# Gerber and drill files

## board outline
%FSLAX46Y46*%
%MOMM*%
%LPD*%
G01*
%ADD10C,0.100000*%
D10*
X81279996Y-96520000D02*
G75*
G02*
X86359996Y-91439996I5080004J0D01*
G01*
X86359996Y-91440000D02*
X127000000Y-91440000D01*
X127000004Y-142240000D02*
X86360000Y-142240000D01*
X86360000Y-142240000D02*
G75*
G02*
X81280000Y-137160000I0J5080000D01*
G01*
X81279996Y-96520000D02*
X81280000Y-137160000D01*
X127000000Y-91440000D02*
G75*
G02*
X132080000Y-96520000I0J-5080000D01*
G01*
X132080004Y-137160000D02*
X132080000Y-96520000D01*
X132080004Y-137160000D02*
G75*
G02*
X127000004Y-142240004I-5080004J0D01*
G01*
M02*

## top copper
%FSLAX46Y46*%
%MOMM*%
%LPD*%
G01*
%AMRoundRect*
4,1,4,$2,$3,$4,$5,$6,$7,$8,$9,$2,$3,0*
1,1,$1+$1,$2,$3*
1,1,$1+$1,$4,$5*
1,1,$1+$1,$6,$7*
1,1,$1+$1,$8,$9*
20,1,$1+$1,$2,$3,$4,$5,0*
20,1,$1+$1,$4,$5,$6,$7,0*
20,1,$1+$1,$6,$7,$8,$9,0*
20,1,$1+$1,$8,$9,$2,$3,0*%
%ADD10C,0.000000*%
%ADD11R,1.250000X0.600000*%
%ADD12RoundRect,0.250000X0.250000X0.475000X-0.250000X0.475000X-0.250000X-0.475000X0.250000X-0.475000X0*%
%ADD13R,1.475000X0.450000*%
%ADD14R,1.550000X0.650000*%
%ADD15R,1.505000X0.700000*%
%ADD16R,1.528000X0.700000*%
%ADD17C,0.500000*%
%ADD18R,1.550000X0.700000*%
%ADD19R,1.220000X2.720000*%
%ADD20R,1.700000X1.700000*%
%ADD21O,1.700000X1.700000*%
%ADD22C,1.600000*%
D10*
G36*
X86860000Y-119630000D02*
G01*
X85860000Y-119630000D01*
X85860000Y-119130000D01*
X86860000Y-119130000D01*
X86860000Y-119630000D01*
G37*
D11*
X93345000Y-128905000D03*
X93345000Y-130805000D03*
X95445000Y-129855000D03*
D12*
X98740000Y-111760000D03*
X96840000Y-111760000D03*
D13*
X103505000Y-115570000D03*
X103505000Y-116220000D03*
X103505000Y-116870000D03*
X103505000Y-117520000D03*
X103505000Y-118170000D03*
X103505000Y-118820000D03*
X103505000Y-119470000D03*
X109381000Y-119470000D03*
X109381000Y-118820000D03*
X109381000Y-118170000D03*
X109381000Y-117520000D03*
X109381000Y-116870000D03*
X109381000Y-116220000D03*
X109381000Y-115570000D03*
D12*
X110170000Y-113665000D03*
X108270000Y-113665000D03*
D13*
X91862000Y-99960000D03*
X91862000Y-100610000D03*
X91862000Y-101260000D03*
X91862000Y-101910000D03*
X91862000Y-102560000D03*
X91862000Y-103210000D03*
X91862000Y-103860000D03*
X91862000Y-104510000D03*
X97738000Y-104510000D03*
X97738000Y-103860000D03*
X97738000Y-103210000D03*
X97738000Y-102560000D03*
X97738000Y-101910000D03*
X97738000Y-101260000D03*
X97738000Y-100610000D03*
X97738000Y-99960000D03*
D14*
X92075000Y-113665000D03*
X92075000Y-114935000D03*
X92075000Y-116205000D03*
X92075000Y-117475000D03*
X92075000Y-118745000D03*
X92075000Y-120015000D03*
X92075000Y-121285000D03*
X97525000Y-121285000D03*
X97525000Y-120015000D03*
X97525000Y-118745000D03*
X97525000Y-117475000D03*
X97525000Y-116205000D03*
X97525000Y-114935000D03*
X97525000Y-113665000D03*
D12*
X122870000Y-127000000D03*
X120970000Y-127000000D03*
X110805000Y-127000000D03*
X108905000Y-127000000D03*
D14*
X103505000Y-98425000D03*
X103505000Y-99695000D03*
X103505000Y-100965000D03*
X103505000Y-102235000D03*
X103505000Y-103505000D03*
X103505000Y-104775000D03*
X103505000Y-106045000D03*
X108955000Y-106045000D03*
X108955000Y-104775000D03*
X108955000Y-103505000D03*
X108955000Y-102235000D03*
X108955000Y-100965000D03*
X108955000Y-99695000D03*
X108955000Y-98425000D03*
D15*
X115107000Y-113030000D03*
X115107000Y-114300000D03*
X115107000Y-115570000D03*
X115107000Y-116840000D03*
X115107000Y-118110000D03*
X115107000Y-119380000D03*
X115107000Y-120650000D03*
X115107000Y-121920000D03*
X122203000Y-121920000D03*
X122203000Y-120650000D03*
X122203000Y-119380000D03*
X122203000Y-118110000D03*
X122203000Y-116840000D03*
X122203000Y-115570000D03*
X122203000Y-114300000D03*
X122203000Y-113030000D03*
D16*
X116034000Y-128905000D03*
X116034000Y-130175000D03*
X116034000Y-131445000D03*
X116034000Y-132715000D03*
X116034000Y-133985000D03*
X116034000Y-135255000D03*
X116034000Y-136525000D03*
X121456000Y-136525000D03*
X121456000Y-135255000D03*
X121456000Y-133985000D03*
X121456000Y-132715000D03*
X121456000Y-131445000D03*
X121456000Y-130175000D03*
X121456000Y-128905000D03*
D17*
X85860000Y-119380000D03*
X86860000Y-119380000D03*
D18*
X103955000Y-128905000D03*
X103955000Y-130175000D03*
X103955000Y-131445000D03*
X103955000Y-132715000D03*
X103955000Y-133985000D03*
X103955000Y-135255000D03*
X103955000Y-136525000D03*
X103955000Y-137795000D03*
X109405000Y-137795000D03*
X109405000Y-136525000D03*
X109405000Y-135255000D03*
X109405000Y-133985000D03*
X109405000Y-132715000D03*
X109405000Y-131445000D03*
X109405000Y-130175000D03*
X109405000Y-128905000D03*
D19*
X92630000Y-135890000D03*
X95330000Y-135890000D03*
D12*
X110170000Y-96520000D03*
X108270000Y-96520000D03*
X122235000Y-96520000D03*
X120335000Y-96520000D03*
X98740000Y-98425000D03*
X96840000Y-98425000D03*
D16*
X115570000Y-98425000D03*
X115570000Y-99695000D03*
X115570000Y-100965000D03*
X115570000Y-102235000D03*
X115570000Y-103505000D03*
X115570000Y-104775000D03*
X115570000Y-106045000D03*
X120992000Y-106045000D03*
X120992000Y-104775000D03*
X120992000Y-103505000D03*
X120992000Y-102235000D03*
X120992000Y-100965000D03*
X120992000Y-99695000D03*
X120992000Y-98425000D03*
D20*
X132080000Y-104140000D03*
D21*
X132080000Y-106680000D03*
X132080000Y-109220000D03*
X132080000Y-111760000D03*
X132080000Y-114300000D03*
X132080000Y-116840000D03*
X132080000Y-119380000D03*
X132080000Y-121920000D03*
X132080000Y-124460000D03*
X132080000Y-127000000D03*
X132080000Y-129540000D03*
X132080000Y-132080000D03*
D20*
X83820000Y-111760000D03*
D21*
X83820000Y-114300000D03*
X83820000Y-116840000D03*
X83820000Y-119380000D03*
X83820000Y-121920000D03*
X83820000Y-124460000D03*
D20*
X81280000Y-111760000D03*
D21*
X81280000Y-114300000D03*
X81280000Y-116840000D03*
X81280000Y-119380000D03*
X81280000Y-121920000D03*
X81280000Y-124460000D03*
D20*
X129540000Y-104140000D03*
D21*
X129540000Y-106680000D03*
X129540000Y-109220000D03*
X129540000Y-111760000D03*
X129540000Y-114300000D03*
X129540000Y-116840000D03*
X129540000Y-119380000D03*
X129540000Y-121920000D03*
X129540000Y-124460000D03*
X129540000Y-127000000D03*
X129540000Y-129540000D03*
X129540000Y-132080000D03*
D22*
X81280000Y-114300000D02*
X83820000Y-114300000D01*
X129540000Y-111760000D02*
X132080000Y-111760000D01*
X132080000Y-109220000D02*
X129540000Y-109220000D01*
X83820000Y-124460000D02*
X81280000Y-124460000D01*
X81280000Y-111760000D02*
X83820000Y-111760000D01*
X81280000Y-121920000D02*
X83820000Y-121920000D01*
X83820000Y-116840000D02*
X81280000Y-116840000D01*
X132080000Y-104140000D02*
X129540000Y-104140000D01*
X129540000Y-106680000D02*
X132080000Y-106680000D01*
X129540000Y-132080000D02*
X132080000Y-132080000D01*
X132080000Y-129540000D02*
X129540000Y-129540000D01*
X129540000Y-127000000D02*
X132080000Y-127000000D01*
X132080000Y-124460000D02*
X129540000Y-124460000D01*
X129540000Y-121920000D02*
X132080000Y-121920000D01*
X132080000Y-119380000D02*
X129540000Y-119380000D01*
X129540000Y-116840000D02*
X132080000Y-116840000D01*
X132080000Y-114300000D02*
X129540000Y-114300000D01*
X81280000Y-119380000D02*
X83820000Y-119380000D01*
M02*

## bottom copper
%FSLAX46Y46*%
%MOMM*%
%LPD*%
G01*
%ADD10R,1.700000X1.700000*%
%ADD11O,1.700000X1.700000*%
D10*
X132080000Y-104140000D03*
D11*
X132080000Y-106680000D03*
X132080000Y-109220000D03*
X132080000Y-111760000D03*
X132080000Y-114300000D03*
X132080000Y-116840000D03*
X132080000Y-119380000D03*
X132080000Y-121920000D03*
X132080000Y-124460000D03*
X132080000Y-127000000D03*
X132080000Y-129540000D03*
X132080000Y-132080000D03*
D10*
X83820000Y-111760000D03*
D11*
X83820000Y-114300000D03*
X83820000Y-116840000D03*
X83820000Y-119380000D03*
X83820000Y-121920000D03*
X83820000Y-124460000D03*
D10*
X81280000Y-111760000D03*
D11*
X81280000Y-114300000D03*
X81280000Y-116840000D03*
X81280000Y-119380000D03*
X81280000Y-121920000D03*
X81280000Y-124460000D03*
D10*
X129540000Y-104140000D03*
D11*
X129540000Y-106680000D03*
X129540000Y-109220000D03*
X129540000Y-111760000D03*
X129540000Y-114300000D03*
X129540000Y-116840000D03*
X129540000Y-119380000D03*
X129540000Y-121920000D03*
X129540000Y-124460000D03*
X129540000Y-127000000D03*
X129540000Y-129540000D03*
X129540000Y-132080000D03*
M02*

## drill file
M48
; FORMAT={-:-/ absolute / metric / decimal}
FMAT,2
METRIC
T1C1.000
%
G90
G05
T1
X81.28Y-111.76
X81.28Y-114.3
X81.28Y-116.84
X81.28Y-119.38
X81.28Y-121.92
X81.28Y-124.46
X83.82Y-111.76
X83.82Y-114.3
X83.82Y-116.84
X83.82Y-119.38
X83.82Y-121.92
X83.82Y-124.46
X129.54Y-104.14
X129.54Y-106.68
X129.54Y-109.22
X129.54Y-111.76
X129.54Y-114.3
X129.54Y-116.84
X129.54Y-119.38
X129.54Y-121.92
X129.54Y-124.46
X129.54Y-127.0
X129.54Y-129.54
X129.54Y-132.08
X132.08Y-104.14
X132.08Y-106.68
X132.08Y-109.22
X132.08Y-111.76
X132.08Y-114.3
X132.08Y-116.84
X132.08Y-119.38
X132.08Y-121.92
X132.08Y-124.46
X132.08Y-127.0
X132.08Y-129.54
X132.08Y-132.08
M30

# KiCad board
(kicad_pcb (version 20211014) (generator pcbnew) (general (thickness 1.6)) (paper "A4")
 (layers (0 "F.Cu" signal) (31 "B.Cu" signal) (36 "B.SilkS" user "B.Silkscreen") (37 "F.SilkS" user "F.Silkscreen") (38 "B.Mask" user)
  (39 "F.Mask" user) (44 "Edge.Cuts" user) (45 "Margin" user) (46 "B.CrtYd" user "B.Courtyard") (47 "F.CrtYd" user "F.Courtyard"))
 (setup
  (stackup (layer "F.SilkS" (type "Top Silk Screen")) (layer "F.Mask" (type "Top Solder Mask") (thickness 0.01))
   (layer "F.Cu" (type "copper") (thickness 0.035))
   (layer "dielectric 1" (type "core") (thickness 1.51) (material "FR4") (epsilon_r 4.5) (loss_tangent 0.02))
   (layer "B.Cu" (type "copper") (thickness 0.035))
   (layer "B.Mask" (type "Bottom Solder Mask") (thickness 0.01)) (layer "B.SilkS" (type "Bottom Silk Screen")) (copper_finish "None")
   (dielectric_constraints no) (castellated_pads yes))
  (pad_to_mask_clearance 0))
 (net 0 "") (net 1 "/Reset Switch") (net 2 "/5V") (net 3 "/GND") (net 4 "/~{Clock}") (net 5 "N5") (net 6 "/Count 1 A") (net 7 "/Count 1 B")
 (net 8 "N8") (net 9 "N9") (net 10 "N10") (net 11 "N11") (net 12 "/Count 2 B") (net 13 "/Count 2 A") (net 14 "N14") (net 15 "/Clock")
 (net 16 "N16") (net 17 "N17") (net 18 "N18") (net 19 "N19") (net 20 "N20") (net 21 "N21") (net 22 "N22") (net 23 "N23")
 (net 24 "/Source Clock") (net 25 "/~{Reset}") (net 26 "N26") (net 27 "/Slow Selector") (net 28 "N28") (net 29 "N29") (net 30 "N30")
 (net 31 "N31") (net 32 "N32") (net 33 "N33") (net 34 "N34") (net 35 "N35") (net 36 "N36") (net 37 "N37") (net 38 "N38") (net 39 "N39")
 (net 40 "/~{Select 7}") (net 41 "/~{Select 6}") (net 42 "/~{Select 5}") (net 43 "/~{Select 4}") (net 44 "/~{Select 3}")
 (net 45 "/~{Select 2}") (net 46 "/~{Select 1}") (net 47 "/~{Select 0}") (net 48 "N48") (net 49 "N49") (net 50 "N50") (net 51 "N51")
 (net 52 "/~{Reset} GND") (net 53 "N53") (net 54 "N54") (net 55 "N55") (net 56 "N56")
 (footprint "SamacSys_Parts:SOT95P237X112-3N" (layer "F.Cu") (at 94.395 129.855)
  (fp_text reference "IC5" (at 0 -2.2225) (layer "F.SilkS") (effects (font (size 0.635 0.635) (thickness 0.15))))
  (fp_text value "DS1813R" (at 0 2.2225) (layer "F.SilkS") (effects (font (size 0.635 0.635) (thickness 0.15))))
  (pad "1" smd rect locked (at -1.05 -0.95 90) (size 0.6 1.25) (layers "F.Cu" "F.Paste" "F.Mask") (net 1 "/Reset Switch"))
  (pad "2" smd rect locked (at -1.05 0.95 90) (size 0.6 1.25) (layers "F.Cu" "F.Paste" "F.Mask") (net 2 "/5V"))
  (pad "3" smd rect locked (at 1.05 0 90) (size 0.6 1.25) (layers "F.Cu" "F.Paste" "F.Mask") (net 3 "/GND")))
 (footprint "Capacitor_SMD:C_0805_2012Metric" (layer "F.Cu") (at 97.79 111.76 180)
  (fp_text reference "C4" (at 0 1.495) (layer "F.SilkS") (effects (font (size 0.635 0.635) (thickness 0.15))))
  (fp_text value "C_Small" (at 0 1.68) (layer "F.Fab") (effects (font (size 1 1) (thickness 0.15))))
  (pad "1" smd roundrect (at -0.95 0 180) (size 1 1.45) (layers "F.Cu" "F.Paste" "F.Mask") (roundrect_rratio 0.25) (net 3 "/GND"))
  (pad "2" smd roundrect (at 0.95 0 180) (size 1 1.45) (layers "F.Cu" "F.Paste" "F.Mask") (roundrect_rratio 0.25) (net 2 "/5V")))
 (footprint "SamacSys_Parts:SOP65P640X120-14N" (layer "F.Cu") (at 106.443 117.52)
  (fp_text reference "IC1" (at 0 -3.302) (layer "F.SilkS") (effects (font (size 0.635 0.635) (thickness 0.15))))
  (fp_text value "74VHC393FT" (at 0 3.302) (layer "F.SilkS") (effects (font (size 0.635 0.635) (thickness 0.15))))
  (pad "1" smd rect (at -2.938 -1.95 90) (size 0.45 1.475) (layers "F.Cu" "F.Paste" "F.Mask") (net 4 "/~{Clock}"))
  (pad "2" smd rect (at -2.938 -1.3 90) (size 0.45 1.475) (layers "F.Cu" "F.Paste" "F.Mask") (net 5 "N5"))
  (pad "3" smd rect (at -2.938 -0.65 90) (size 0.45 1.475) (layers "F.Cu" "F.Paste" "F.Mask") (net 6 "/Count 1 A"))
  (pad "4" smd rect (at -2.938 0 90) (size 0.45 1.475) (layers "F.Cu" "F.Paste" "F.Mask") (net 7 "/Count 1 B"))
  (pad "5" smd rect (at -2.938 0.65 90) (size 0.45 1.475) (layers "F.Cu" "F.Paste" "F.Mask") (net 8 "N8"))
  (pad "6" smd rect (at -2.938 1.3 90) (size 0.45 1.475) (layers "F.Cu" "F.Paste" "F.Mask") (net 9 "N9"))
  (pad "7" smd rect (at -2.938 1.95 90) (size 0.45 1.475) (layers "F.Cu" "F.Paste" "F.Mask") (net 3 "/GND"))
  (pad "8" smd rect (at 2.938 1.95 90) (size 0.45 1.475) (layers "F.Cu" "F.Paste" "F.Mask") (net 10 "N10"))
  (pad "9" smd rect (at 2.938 1.3 90) (size 0.45 1.475) (layers "F.Cu" "F.Paste" "F.Mask") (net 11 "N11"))
  (pad "10" smd rect (at 2.938 0.65 90) (size 0.45 1.475) (layers "F.Cu" "F.Paste" "F.Mask") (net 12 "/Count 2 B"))
  (pad "11" smd rect (at 2.938 0 90) (size 0.45 1.475) (layers "F.Cu" "F.Paste" "F.Mask") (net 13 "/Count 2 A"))
  (pad "12" smd rect (at 2.938 -0.65 90) (size 0.45 1.475) (layers "F.Cu" "F.Paste" "F.Mask") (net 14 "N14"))
  (pad "13" smd rect (at 2.938 -1.3 90) (size 0.45 1.475) (layers "F.Cu" "F.Paste" "F.Mask") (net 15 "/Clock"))
  (pad "14" smd rect (at 2.938 -1.95 90) (size 0.45 1.475) (layers "F.Cu" "F.Paste" "F.Mask") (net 2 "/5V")))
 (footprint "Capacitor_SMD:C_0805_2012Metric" (layer "F.Cu") (at 109.22 113.665 180)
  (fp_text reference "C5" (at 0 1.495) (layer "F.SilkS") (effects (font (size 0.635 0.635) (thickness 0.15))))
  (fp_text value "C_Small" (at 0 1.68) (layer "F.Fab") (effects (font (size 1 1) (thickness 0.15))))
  (pad "1" smd roundrect (at -0.95 0 180) (size 1 1.45) (layers "F.Cu" "F.Paste" "F.Mask") (roundrect_rratio 0.25) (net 3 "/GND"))
  (pad "2" smd roundrect (at 0.95 0 180) (size 1 1.45) (layers "F.Cu" "F.Paste" "F.Mask") (roundrect_rratio 0.25) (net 2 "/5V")))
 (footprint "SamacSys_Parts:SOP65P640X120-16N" (layer "F.Cu") (at 94.8 102.235)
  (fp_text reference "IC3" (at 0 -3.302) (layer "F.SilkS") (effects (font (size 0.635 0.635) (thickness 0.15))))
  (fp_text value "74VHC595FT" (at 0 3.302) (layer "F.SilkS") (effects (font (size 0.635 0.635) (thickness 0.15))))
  (pad "1" smd rect (at -2.938 -2.275 90) (size 0.45 1.475) (layers "F.Cu" "F.Paste" "F.Mask") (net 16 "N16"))
  (pad "2" smd rect (at -2.938 -1.625 90) (size 0.45 1.475) (layers "F.Cu" "F.Paste" "F.Mask") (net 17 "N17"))
  (pad "3" smd rect (at -2.938 -0.975 90) (size 0.45 1.475) (layers "F.Cu" "F.Paste" "F.Mask") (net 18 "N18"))
  (pad "4" smd rect (at -2.938 -0.325 90) (size 0.45 1.475) (layers "F.Cu" "F.Paste" "F.Mask") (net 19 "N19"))
  (pad "5" smd rect (at -2.938 0.325 90) (size 0.45 1.475) (layers "F.Cu" "F.Paste" "F.Mask") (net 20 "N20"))
  (pad "6" smd rect (at -2.938 0.975 90) (size 0.45 1.475) (layers "F.Cu" "F.Paste" "F.Mask") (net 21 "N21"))
  (pad "7" smd rect (at -2.938 1.625 90) (size 0.45 1.475) (layers "F.Cu" "F.Paste" "F.Mask") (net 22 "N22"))
  (pad "8" smd rect (at -2.938 2.275 90) (size 0.45 1.475) (layers "F.Cu" "F.Paste" "F.Mask") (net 3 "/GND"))
  (pad "9" smd rect (at 2.938 2.275 90) (size 0.45 1.475) (layers "F.Cu" "F.Paste" "F.Mask") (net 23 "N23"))
  (pad "10" smd rect (at 2.938 1.625 90) (size 0.45 1.475) (layers "F.Cu" "F.Paste" "F.Mask") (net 1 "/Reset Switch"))
  (pad "11" smd rect (at 2.938 0.975 90) (size 0.45 1.475) (layers "F.Cu" "F.Paste" "F.Mask") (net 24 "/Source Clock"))
  (pad "12" smd rect (at 2.938 0.325 90) (size 0.45 1.475) (layers "F.Cu" "F.Paste" "F.Mask") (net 24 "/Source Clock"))
  (pad "13" smd rect (at 2.938 -0.325 90) (size 0.45 1.475) (layers "F.Cu" "F.Paste" "F.Mask") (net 3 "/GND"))
  (pad "14" smd rect (at 2.938 -0.975 90) (size 0.45 1.475) (layers "F.Cu" "F.Paste" "F.Mask") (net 1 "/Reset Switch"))
  (pad "15" smd rect (at 2.938 -1.625 90) (size 0.45 1.475) (layers "F.Cu" "F.Paste" "F.Mask") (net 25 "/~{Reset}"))
  (pad "16" smd rect (at 2.938 -2.275 90) (size 0.45 1.475) (layers "F.Cu" "F.Paste" "F.Mask") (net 2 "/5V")))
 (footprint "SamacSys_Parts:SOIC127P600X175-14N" (layer "F.Cu") (at 94.8 117.475)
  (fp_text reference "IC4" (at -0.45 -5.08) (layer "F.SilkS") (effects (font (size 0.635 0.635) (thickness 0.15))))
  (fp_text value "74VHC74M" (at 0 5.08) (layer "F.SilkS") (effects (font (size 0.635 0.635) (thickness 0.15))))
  (pad "1" smd rect locked (at -2.725 -3.81 90) (size 0.65 1.55) (layers "F.Cu" "F.Paste" "F.Mask") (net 19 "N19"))
  (pad "2" smd rect locked (at -2.725 -2.54 90) (size 0.65 1.55) (layers "F.Cu" "F.Paste" "F.Mask") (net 4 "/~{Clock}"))
  (pad "3" smd rect locked (at -2.725 -1.27 90) (size 0.65 1.55) (layers "F.Cu" "F.Paste" "F.Mask") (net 24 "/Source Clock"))
  (pad "4" smd rect locked (at -2.725 0 90) (size 0.65 1.55) (layers "F.Cu" "F.Paste" "F.Mask") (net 2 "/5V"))
  (pad "5" smd rect locked (at -2.725 1.27 90) (size 0.65 1.55) (layers "F.Cu" "F.Paste" "F.Mask") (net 15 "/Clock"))
  (pad "6" smd rect locked (at -2.725 2.54 90) (size 0.65 1.55) (layers "F.Cu" "F.Paste" "F.Mask") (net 4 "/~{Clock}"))
  (pad "7" smd rect locked (at -2.725 3.81 90) (size 0.65 1.55) (layers "F.Cu" "F.Paste" "F.Mask") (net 3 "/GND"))
  (pad "8" smd rect locked (at 2.725 3.81 90) (size 0.65 1.55) (layers "F.Cu" "F.Paste" "F.Mask") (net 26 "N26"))
  (pad "9" smd rect locked (at 2.725 2.54 90) (size 0.65 1.55) (layers "F.Cu" "F.Paste" "F.Mask") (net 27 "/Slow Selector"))
  (pad "10" smd rect locked (at 2.725 1.27 90) (size 0.65 1.55) (layers "F.Cu" "F.Paste" "F.Mask") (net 2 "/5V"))
  (pad "11" smd rect locked (at 2.725 0 90) (size 0.65 1.55) (layers "F.Cu" "F.Paste" "F.Mask") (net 9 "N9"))
  (pad "12" smd rect locked (at 2.725 -1.27 90) (size 0.65 1.55) (layers "F.Cu" "F.Paste" "F.Mask") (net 26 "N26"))
  (pad "13" smd rect locked (at 2.725 -2.54 90) (size 0.65 1.55) (layers "F.Cu" "F.Paste" "F.Mask") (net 19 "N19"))
  (pad "14" smd rect locked (at 2.725 -3.81 90) (size 0.65 1.55) (layers "F.Cu" "F.Paste" "F.Mask") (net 2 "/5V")))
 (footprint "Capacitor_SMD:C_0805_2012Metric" (layer "F.Cu") (at 121.92 127 180)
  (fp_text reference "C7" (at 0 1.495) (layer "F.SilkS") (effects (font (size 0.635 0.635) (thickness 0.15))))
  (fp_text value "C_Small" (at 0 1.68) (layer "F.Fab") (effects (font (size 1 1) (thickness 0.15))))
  (pad "1" smd roundrect (at -0.95 0 180) (size 1 1.45) (layers "F.Cu" "F.Paste" "F.Mask") (roundrect_rratio 0.25) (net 3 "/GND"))
  (pad "2" smd roundrect (at 0.95 0 180) (size 1 1.45) (layers "F.Cu" "F.Paste" "F.Mask") (roundrect_rratio 0.25) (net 2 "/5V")))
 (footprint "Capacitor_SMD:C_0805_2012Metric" (layer "F.Cu") (at 109.855 127 180)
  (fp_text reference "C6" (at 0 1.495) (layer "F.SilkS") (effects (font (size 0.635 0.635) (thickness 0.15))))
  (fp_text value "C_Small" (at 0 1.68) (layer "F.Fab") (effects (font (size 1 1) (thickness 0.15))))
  (pad "1" smd roundrect (at -0.95 0 180) (size 1 1.45) (layers "F.Cu" "F.Paste" "F.Mask") (roundrect_rratio 0.25) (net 3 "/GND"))
  (pad "2" smd roundrect (at 0.95 0 180) (size 1 1.45) (layers "F.Cu" "F.Paste" "F.Mask") (roundrect_rratio 0.25) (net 2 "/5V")))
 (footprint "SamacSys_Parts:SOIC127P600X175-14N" (layer "F.Cu") (at 106.23 102.235)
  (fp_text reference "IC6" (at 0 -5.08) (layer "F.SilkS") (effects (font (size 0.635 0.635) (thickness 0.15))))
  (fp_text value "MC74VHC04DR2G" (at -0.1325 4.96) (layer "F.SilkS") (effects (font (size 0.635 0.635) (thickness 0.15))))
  (pad "1" smd rect locked (at -2.725 -3.81 90) (size 0.65 1.55) (layers "F.Cu" "F.Paste" "F.Mask") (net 21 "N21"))
  (pad "2" smd rect locked (at -2.725 -2.54 90) (size 0.65 1.55) (layers "F.Cu" "F.Paste" "F.Mask") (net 5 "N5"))
  (pad "3" smd rect locked (at -2.725 -1.27 90) (size 0.65 1.55) (layers "F.Cu" "F.Paste" "F.Mask") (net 22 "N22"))
  (pad "4" smd rect locked (at -2.725 0 90) (size 0.65 1.55) (layers "F.Cu" "F.Paste" "F.Mask") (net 14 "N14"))
  (pad "5" smd rect locked (at -2.725 1.27 90) (size 0.65 1.55) (layers "F.Cu" "F.Paste" "F.Mask") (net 3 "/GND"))
  (pad "6" smd rect locked (at -2.725 2.54 90) (size 0.65 1.55) (layers "F.Cu" "F.Paste" "F.Mask") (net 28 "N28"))
  (pad "7" smd rect locked (at -2.725 3.81 90) (size 0.65 1.55) (layers "F.Cu" "F.Paste" "F.Mask") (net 3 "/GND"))
  (pad "8" smd rect locked (at 2.725 3.81 90) (size 0.65 1.55) (layers "F.Cu" "F.Paste" "F.Mask") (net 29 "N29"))
  (pad "9" smd rect locked (at 2.725 2.54 90) (size 0.65 1.55) (layers "F.Cu" "F.Paste" "F.Mask") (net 3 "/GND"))
  (pad "10" smd rect locked (at 2.725 1.27 90) (size 0.65 1.55) (layers "F.Cu" "F.Paste" "F.Mask") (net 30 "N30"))
  (pad "11" smd rect locked (at 2.725 0 90) (size 0.65 1.55) (layers "F.Cu" "F.Paste" "F.Mask") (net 3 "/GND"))
  (pad "12" smd rect locked (at 2.725 -1.27 90) (size 0.65 1.55) (layers "F.Cu" "F.Paste" "F.Mask") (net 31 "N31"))
  (pad "13" smd rect locked (at 2.725 -2.54 90) (size 0.65 1.55) (layers "F.Cu" "F.Paste" "F.Mask") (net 3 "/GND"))
  (pad "14" smd rect locked (at 2.725 -3.81 90) (size 0.65 1.55) (layers "F.Cu" "F.Paste" "F.Mask") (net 2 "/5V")))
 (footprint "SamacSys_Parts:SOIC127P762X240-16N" (layer "F.Cu") (at 118.655 117.475)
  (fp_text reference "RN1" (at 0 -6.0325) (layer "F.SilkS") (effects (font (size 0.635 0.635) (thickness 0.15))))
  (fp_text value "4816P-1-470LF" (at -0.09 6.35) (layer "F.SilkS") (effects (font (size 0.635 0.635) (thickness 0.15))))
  (pad "1" smd rect (at -3.548 -4.445 90) (size 0.7 1.505) (layers "F.Cu" "F.Paste" "F.Mask") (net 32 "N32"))
  (pad "2" smd rect (at -3.548 -3.175 90) (size 0.7 1.505) (layers "F.Cu" "F.Paste" "F.Mask") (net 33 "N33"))
  (pad "3" smd rect (at -3.548 -1.905 90) (size 0.7 1.505) (layers "F.Cu" "F.Paste" "F.Mask") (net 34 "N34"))
  (pad "4" smd rect (at -3.548 -0.635 90) (size 0.7 1.505) (layers "F.Cu" "F.Paste" "F.Mask") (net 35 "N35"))
  (pad "5" smd rect (at -3.548 0.635 90) (size 0.7 1.505) (layers "F.Cu" "F.Paste" "F.Mask") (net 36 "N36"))
  (pad "6" smd rect (at -3.548 1.905 90) (size 0.7 1.505) (layers "F.Cu" "F.Paste" "F.Mask") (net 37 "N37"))
  (pad "7" smd rect (at -3.548 3.175 90) (size 0.7 1.505) (layers "F.Cu" "F.Paste" "F.Mask") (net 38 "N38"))
  (pad "8" smd rect (at -3.548 4.445 90) (size 0.7 1.505) (layers "F.Cu" "F.Paste" "F.Mask") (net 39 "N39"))
  (pad "9" smd rect (at 3.548 4.445 90) (size 0.7 1.505) (layers "F.Cu" "F.Paste" "F.Mask") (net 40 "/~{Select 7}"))
  (pad "10" smd rect (at 3.548 3.175 90) (size 0.7 1.505) (layers "F.Cu" "F.Paste" "F.Mask") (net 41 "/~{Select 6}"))
  (pad "11" smd rect (at 3.548 1.905 90) (size 0.7 1.505) (layers "F.Cu" "F.Paste" "F.Mask") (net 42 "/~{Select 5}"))
  (pad "12" smd rect (at 3.548 0.635 90) (size 0.7 1.505) (layers "F.Cu" "F.Paste" "F.Mask") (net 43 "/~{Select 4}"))
  (pad "13" smd rect (at 3.548 -0.635 90) (size 0.7 1.505) (layers "F.Cu" "F.Paste" "F.Mask") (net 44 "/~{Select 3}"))
  (pad "14" smd rect (at 3.548 -1.905 90) (size 0.7 1.505) (layers "F.Cu" "F.Paste" "F.Mask") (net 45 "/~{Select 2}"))
  (pad "15" smd rect (at 3.548 -3.175 90) (size 0.7 1.505) (layers "F.Cu" "F.Paste" "F.Mask") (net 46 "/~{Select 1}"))
  (pad "16" smd rect (at 3.548 -4.445 90) (size 0.7 1.505) (layers "F.Cu" "F.Paste" "F.Mask") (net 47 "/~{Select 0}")))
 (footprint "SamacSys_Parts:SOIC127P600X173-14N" (layer "F.Cu") (at 118.745 132.715)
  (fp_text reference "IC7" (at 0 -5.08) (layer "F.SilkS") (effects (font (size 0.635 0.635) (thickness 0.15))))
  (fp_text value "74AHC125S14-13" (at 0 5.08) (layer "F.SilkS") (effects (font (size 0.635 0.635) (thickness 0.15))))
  (pad "1" smd rect (at -2.711 -3.81 90) (size 0.7 1.528) (layers "F.Cu" "F.Paste" "F.Mask") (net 3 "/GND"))
  (pad "2" smd rect (at -2.711 -2.54 90) (size 0.7 1.528) (layers "F.Cu" "F.Paste" "F.Mask") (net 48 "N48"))
  (pad "3" smd rect (at -2.711 -1.27 90) (size 0.7 1.528) (layers "F.Cu" "F.Paste" "F.Mask") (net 33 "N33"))
  (pad "4" smd rect (at -2.711 0 90) (size 0.7 1.528) (layers "F.Cu" "F.Paste" "F.Mask") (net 3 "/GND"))
  (pad "5" smd rect (at -2.711 1.27 90) (size 0.7 1.528) (layers "F.Cu" "F.Paste" "F.Mask") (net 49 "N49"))
  (pad "6" smd rect (at -2.711 2.54 90) (size 0.7 1.528) (layers "F.Cu" "F.Paste" "F.Mask") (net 35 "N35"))
  (pad "7" smd rect (at -2.711 3.81 90) (size 0.7 1.528) (layers "F.Cu" "F.Paste" "F.Mask") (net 3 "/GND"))
  (pad "8" smd rect (at 2.711 3.81 90) (size 0.7 1.528) (layers "F.Cu" "F.Paste" "F.Mask") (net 37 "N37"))
  (pad "9" smd rect (at 2.711 2.54 90) (size 0.7 1.528) (layers "F.Cu" "F.Paste" "F.Mask") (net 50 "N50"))
  (pad "10" smd rect (at 2.711 1.27 90) (size 0.7 1.528) (layers "F.Cu" "F.Paste" "F.Mask") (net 3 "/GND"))
  (pad "11" smd rect (at 2.711 0 90) (size 0.7 1.528) (layers "F.Cu" "F.Paste" "F.Mask") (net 39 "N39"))
  (pad "12" smd rect (at 2.711 -1.27 90) (size 0.7 1.528) (layers "F.Cu" "F.Paste" "F.Mask") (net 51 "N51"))
  (pad "13" smd rect (at 2.711 -2.54 90) (size 0.7 1.528) (layers "F.Cu" "F.Paste" "F.Mask") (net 3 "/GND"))
  (pad "14" smd rect (at 2.711 -3.81 90) (size 0.7 1.528) (layers "F.Cu" "F.Paste" "F.Mask") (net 2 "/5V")))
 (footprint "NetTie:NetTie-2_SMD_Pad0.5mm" (layer "F.Cu") (at 86.36 119.38)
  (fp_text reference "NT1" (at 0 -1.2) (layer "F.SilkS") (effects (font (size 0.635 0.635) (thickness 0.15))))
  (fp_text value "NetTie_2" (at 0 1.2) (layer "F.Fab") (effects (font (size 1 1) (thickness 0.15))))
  (fp_poly (pts (xy -0.5 -0.25) (xy 0.5 -0.25) (xy 0.5 0.25) (xy -0.5 0.25)) (layer "F.Cu") (width 0) (fill solid))
  (pad "1" smd circle (at -0.5 0) (size 0.5 0.5) (layers "F.Cu") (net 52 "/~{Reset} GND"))
  (pad "2" smd circle (at 0.5 0) (size 0.5 0.5) (layers "F.Cu") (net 3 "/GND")))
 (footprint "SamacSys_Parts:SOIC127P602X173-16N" (layer "F.Cu") (at 106.68 133.35)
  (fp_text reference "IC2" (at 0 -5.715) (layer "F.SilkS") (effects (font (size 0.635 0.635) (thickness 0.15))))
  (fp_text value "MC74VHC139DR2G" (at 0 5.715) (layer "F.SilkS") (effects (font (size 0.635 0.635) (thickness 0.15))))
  (pad "1" smd rect (at -2.725 -4.445 90) (size 0.7 1.55) (layers "F.Cu" "F.Paste" "F.Mask") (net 3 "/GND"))
  (pad "2" smd rect (at -2.725 -3.175 90) (size 0.7 1.55) (layers "F.Cu" "F.Paste" "F.Mask") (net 6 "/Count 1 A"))
  (pad "3" smd rect (at -2.725 -1.905 90) (size 0.7 1.55) (layers "F.Cu" "F.Paste" "F.Mask") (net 7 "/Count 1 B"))
  (pad "4" smd rect (at -2.725 -0.635 90) (size 0.7 1.55) (layers "F.Cu" "F.Paste" "F.Mask") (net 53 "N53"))
  (pad "5" smd rect (at -2.725 0.635 90) (size 0.7 1.55) (layers "F.Cu" "F.Paste" "F.Mask") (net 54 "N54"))
  (pad "6" smd rect (at -2.725 1.905 90) (size 0.7 1.55) (layers "F.Cu" "F.Paste" "F.Mask") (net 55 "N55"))
  (pad "7" smd rect (at -2.725 3.175 90) (size 0.7 1.55) (layers "F.Cu" "F.Paste" "F.Mask") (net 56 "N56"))
  (pad "8" smd rect (at -2.725 4.445 90) (size 0.7 1.55) (layers "F.Cu" "F.Paste" "F.Mask") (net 3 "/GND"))
  (pad "9" smd rect (at 2.725 4.445 90) (size 0.7 1.55) (layers "F.Cu" "F.Paste" "F.Mask") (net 51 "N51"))
  (pad "10" smd rect (at 2.725 3.175 90) (size 0.7 1.55) (layers "F.Cu" "F.Paste" "F.Mask") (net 50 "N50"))
  (pad "11" smd rect (at 2.725 1.905 90) (size 0.7 1.55) (layers "F.Cu" "F.Paste" "F.Mask") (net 49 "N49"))
  (pad "12" smd rect (at 2.725 0.635 90) (size 0.7 1.55) (layers "F.Cu" "F.Paste" "F.Mask") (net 48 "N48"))
  (pad "13" smd rect (at 2.725 -0.635 90) (size 0.7 1.55) (layers "F.Cu" "F.Paste" "F.Mask") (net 12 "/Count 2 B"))
  (pad "14" smd rect (at 2.725 -1.905 90) (size 0.7 1.55) (layers "F.Cu" "F.Paste" "F.Mask") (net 13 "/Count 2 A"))
  (pad "15" smd rect (at 2.725 -3.175 90) (size 0.7 1.55) (layers "F.Cu" "F.Paste" "F.Mask") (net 3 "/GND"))
  (pad "16" smd rect (at 2.725 -4.445 90) (size 0.7 1.55) (layers "F.Cu" "F.Paste" "F.Mask") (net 2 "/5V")))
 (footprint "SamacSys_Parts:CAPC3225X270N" (layer "F.Cu") (at 93.98 135.89)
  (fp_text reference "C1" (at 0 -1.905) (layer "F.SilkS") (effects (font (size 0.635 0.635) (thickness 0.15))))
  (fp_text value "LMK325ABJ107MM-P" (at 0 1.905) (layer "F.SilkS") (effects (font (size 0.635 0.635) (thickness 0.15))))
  (pad "1" smd rect locked (at -1.35 0) (size 1.22 2.72) (layers "F.Cu" "F.Paste" "F.Mask") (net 2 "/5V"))
  (pad "2" smd rect locked (at 1.35 0) (size 1.22 2.72) (layers "F.Cu" "F.Paste" "F.Mask") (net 3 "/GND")))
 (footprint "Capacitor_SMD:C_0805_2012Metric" (layer "F.Cu") (at 109.22 96.52 180)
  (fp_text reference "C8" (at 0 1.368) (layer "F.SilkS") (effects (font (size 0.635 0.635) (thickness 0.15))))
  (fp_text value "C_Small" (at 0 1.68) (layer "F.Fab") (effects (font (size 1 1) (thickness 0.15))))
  (pad "1" smd roundrect (at -0.95 0 180) (size 1 1.45) (layers "F.Cu" "F.Paste" "F.Mask") (roundrect_rratio 0.25) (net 3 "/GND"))
  (pad "2" smd roundrect (at 0.95 0 180) (size 1 1.45) (layers "F.Cu" "F.Paste" "F.Mask") (roundrect_rratio 0.25) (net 2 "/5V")))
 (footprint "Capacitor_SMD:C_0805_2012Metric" (layer "F.Cu") (at 121.285 96.52 180)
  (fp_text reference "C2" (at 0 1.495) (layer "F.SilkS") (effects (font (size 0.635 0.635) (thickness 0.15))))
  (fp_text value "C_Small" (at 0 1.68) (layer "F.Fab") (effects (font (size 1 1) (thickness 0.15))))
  (pad "1" smd roundrect (at -0.95 0 180) (size 1 1.45) (layers "F.Cu" "F.Paste" "F.Mask") (roundrect_rratio 0.25) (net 3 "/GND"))
  (pad "2" smd roundrect (at 0.95 0 180) (size 1 1.45) (layers "F.Cu" "F.Paste" "F.Mask") (roundrect_rratio 0.25) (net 2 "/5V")))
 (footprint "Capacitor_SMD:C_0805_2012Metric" (layer "F.Cu") (at 97.79 98.425 180)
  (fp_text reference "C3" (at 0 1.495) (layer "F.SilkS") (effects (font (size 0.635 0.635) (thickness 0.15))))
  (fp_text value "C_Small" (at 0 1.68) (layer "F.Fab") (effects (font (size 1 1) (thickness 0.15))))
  (pad "1" smd roundrect (at -0.95 0 180) (size 1 1.45) (layers "F.Cu" "F.Paste" "F.Mask") (roundrect_rratio 0.25) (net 3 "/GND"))
  (pad "2" smd roundrect (at 0.95 0 180) (size 1 1.45) (layers "F.Cu" "F.Paste" "F.Mask") (roundrect_rratio 0.25) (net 2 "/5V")))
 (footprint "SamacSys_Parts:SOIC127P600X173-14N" (layer "F.Cu") (at 118.281 102.235)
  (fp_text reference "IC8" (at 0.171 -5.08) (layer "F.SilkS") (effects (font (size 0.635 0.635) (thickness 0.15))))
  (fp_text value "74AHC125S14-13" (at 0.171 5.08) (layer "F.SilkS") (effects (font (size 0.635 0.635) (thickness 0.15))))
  (pad "1" smd rect (at -2.711 -3.81 90) (size 0.7 1.528) (layers "F.Cu" "F.Paste" "F.Mask") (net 3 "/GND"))
  (pad "2" smd rect (at -2.711 -2.54 90) (size 0.7 1.528) (layers "F.Cu" "F.Paste" "F.Mask") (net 53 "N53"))
  (pad "3" smd rect (at -2.711 -1.27 90) (size 0.7 1.528) (layers "F.Cu" "F.Paste" "F.Mask") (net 32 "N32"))
  (pad "4" smd rect (at -2.711 0 90) (size 0.7 1.528) (layers "F.Cu" "F.Paste" "F.Mask") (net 3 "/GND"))
  (pad "5" smd rect (at -2.711 1.27 90) (size 0.7 1.528) (layers "F.Cu" "F.Paste" "F.Mask") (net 54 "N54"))
  (pad "6" smd rect (at -2.711 2.54 90) (size 0.7 1.528) (layers "F.Cu" "F.Paste" "F.Mask") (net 34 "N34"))
  (pad "7" smd rect (at -2.711 3.81 90) (size 0.7 1.528) (layers "F.Cu" "F.Paste" "F.Mask") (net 3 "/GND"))
  (pad "8" smd rect (at 2.711 3.81 90) (size 0.7 1.528) (layers "F.Cu" "F.Paste" "F.Mask") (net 36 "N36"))
  (pad "9" smd rect (at 2.711 2.54 90) (size 0.7 1.528) (layers "F.Cu" "F.Paste" "F.Mask") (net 55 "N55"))
  (pad "10" smd rect (at 2.711 1.27 90) (size 0.7 1.528) (layers "F.Cu" "F.Paste" "F.Mask") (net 3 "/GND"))
  (pad "11" smd rect (at 2.711 0 90) (size 0.7 1.528) (layers "F.Cu" "F.Paste" "F.Mask") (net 38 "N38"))
  (pad "12" smd rect (at 2.711 -1.27 90) (size 0.7 1.528) (layers "F.Cu" "F.Paste" "F.Mask") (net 56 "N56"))
  (pad "13" smd rect (at 2.711 -2.54 90) (size 0.7 1.528) (layers "F.Cu" "F.Paste" "F.Mask") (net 3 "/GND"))
  (pad "14" smd rect (at 2.711 -3.81 90) (size 0.7 1.528) (layers "F.Cu" "F.Paste" "F.Mask") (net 2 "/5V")))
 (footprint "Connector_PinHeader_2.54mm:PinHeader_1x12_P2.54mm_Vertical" (layer "B.Cu") (at 132.08 104.14 180)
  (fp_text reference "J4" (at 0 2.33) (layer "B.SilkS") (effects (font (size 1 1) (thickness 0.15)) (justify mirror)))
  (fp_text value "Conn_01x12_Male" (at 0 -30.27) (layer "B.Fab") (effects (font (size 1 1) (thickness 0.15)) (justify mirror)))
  (pad "1" thru_hole rect (at 0 0 180) (size 1.7 1.7) (drill 1) (layers *.Cu *.Mask) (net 25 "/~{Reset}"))
  (pad "2" thru_hole oval (at 0 -2.54 180) (size 1.7 1.7) (drill 1) (layers *.Cu *.Mask) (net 27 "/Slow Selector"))
  (pad "3" thru_hole oval (at 0 -5.08 180) (size 1.7 1.7) (drill 1) (layers *.Cu *.Mask) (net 15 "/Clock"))
  (pad "4" thru_hole oval (at 0 -7.62 180) (size 1.7 1.7) (drill 1) (layers *.Cu *.Mask) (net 4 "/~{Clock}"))
  (pad "5" thru_hole oval (at 0 -10.16 180) (size 1.7 1.7) (drill 1) (layers *.Cu *.Mask) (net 47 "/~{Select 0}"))
  (pad "6" thru_hole oval (at 0 -12.7 180) (size 1.7 1.7) (drill 1) (layers *.Cu *.Mask) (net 46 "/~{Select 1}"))
  (pad "7" thru_hole oval (at 0 -15.24 180) (size 1.7 1.7) (drill 1) (layers *.Cu *.Mask) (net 45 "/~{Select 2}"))
  (pad "8" thru_hole oval (at 0 -17.78 180) (size 1.7 1.7) (drill 1) (layers *.Cu *.Mask) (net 44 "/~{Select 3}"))
  (pad "9" thru_hole oval (at 0 -20.32 180) (size 1.7 1.7) (drill 1) (layers *.Cu *.Mask) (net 43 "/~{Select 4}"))
  (pad "10" thru_hole oval (at 0 -22.86 180) (size 1.7 1.7) (drill 1) (layers *.Cu *.Mask) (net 42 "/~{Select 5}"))
  (pad "11" thru_hole oval (at 0 -25.4 180) (size 1.7 1.7) (drill 1) (layers *.Cu *.Mask) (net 41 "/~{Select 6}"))
  (pad "12" thru_hole oval (at 0 -27.94 180) (size 1.7 1.7) (drill 1) (layers *.Cu *.Mask) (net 40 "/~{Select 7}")))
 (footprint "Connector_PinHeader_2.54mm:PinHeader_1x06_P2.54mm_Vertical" (layer "B.Cu") (at 83.82 111.76 180)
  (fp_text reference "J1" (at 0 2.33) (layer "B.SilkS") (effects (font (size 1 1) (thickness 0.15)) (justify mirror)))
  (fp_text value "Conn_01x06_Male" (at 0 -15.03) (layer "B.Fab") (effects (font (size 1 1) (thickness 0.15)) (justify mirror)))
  (pad "1" thru_hole rect (at 0 0 180) (size 1.7 1.7) (drill 1) (layers *.Cu *.Mask) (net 3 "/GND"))
  (pad "2" thru_hole oval (at 0 -2.54 180) (size 1.7 1.7) (drill 1) (layers *.Cu *.Mask) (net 2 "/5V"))
  (pad "3" thru_hole oval (at 0 -5.08 180) (size 1.7 1.7) (drill 1) (layers *.Cu *.Mask) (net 24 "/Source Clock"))
  (pad "4" thru_hole oval (at 0 -7.62 180) (size 1.7 1.7) (drill 1) (layers *.Cu *.Mask) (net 52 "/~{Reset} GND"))
  (pad "5" thru_hole oval (at 0 -10.16 180) (size 1.7 1.7) (drill 1) (layers *.Cu *.Mask) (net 1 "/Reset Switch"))
  (pad "6" thru_hole oval (at 0 -12.7 180) (size 1.7 1.7) (drill 1) (layers *.Cu *.Mask) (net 3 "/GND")))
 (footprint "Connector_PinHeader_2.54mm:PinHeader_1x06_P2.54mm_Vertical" (layer "B.Cu") (at 81.28 111.76 180)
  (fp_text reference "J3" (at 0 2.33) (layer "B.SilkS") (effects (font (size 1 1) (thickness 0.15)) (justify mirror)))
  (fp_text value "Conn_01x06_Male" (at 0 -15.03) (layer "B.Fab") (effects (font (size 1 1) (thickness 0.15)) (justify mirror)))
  (pad "1" thru_hole rect (at 0 0 180) (size 1.7 1.7) (drill 1) (layers *.Cu *.Mask) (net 3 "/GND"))
  (pad "2" thru_hole oval (at 0 -2.54 180) (size 1.7 1.7) (drill 1) (layers *.Cu *.Mask) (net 2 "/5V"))
  (pad "3" thru_hole oval (at 0 -5.08 180) (size 1.7 1.7) (drill 1) (layers *.Cu *.Mask) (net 24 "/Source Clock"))
  (pad "4" thru_hole oval (at 0 -7.62 180) (size 1.7 1.7) (drill 1) (layers *.Cu *.Mask) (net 52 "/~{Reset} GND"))
  (pad "5" thru_hole oval (at 0 -10.16 180) (size 1.7 1.7) (drill 1) (layers *.Cu *.Mask) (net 1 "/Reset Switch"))
  (pad "6" thru_hole oval (at 0 -12.7 180) (size 1.7 1.7) (drill 1) (layers *.Cu *.Mask) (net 3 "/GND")))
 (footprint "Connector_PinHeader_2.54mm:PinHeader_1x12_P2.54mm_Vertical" (layer "B.Cu") (at 129.54 104.14 180)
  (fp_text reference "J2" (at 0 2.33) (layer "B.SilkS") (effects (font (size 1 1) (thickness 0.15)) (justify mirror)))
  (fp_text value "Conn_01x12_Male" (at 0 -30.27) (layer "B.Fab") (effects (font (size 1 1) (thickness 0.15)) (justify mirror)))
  (pad "1" thru_hole rect (at 0 0 180) (size 1.7 1.7) (drill 1) (layers *.Cu *.Mask) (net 25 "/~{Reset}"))
  (pad "2" thru_hole oval (at 0 -2.54 180) (size 1.7 1.7) (drill 1) (layers *.Cu *.Mask) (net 27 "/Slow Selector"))
  (pad "3" thru_hole oval (at 0 -5.08 180) (size 1.7 1.7) (drill 1) (layers *.Cu *.Mask) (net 15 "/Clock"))
  (pad "4" thru_hole oval (at 0 -7.62 180) (size 1.7 1.7) (drill 1) (layers *.Cu *.Mask) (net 4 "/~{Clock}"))
  (pad "5" thru_hole oval (at 0 -10.16 180) (size 1.7 1.7) (drill 1) (layers *.Cu *.Mask) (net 47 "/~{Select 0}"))
  (pad "6" thru_hole oval (at 0 -12.7 180) (size 1.7 1.7) (drill 1) (layers *.Cu *.Mask) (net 46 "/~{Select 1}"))
  (pad "7" thru_hole oval (at 0 -15.24 180) (size 1.7 1.7) (drill 1) (layers *.Cu *.Mask) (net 45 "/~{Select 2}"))
  (pad "8" thru_hole oval (at 0 -17.78 180) (size 1.7 1.7) (drill 1) (layers *.Cu *.Mask) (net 44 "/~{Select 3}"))
  (pad "9" thru_hole oval (at 0 -20.32 180) (size 1.7 1.7) (drill 1) (layers *.Cu *.Mask) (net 43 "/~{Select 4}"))
  (pad "10" thru_hole oval (at 0 -22.86 180) (size 1.7 1.7) (drill 1) (layers *.Cu *.Mask) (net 42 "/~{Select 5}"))
  (pad "11" thru_hole oval (at 0 -25.4 180) (size 1.7 1.7) (drill 1) (layers *.Cu *.Mask) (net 41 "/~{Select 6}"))
  (pad "12" thru_hole oval (at 0 -27.94 180) (size 1.7 1.7) (drill 1) (layers *.Cu *.Mask) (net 40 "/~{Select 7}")))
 (gr_arc (start 81.279996 96.52) (mid 82.767894 92.927898) (end 86.359996 91.44) (layer "Edge.Cuts") (width 0.1))
 (gr_line (start 86.359996 91.44) (end 127 91.44) (layer "Edge.Cuts") (width 0.1))
 (gr_line (start 127.000004 142.24) (end 86.36 142.24) (layer "Edge.Cuts") (width 0.1))
 (gr_arc (start 86.36 142.24) (mid 82.767898 140.752102) (end 81.28 137.16) (layer "Edge.Cuts") (width 0.1))
 (gr_line (start 81.279996 96.52) (end 81.28 137.16) (layer "Edge.Cuts") (width 0.1))
 (gr_arc (start 127 91.44) (mid 130.592102 92.927898) (end 132.08 96.52) (layer "Edge.Cuts") (width 0.1))
 (gr_line (start 132.080004 137.16) (end 132.08 96.52) (layer "Edge.Cuts") (width 0.1))
 (gr_arc (start 132.080004 137.16) (mid 130.592106 140.752102) (end 127.000004 142.24) (layer "Edge.Cuts") (width 0.1))
 (segment (start 81.28 114.3) (end 83.82 114.3) (width 1.6) (layer "F.Cu") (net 2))
 (segment (start 129.54 111.76) (end 132.08 111.76) (width 1.6) (layer "F.Cu") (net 4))
 (segment (start 132.08 109.22) (end 129.54 109.22) (width 1.6) (layer "F.Cu") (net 15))
 (segment (start 83.82 124.46) (end 81.28 124.46) (width 1.6) (layer "F.Cu") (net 3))
 (segment (start 81.28 111.76) (end 83.82 111.76) (width 1.6) (layer "F.Cu") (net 3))
 (segment (start 81.28 121.92) (end 83.82 121.92) (width 1.6) (layer "F.Cu") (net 1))
 (segment (start 83.82 116.84) (end 81.28 116.84) (width 1.6) (layer "F.Cu") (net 24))
 (segment (start 132.08 104.14) (end 129.54 104.14) (width 1.6) (layer "F.Cu") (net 25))
 (segment (start 129.54 106.68) (end 132.08 106.68) (width 1.6) (layer "F.Cu") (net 27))
 (segment (start 129.54 132.08) (end 132.08 132.08) (width 1.6) (layer "F.Cu") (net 40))
 (segment (start 132.08 129.54) (end 129.54 129.54) (width 1.6) (layer "F.Cu") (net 41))
 (segment (start 129.54 127) (end 132.08 127) (width 1.6) (layer "F.Cu") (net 42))
 (segment (start 132.08 124.46) (end 129.54 124.46) (width 1.6) (layer "F.Cu") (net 43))
 (segment (start 129.54 121.92) (end 132.08 121.92) (width 1.6) (layer "F.Cu") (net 44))
 (segment (start 132.08 119.38) (end 129.54 119.38) (width 1.6) (layer "F.Cu") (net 45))
 (segment (start 129.54 116.84) (end 132.08 116.84) (width 1.6) (layer "F.Cu") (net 46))
 (segment (start 132.08 114.3) (end 129.54 114.3) (width 1.6) (layer "F.Cu") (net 47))
 (segment (start 81.28 119.38) (end 83.82 119.38) (width 1.6) (layer "F.Cu") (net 52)))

